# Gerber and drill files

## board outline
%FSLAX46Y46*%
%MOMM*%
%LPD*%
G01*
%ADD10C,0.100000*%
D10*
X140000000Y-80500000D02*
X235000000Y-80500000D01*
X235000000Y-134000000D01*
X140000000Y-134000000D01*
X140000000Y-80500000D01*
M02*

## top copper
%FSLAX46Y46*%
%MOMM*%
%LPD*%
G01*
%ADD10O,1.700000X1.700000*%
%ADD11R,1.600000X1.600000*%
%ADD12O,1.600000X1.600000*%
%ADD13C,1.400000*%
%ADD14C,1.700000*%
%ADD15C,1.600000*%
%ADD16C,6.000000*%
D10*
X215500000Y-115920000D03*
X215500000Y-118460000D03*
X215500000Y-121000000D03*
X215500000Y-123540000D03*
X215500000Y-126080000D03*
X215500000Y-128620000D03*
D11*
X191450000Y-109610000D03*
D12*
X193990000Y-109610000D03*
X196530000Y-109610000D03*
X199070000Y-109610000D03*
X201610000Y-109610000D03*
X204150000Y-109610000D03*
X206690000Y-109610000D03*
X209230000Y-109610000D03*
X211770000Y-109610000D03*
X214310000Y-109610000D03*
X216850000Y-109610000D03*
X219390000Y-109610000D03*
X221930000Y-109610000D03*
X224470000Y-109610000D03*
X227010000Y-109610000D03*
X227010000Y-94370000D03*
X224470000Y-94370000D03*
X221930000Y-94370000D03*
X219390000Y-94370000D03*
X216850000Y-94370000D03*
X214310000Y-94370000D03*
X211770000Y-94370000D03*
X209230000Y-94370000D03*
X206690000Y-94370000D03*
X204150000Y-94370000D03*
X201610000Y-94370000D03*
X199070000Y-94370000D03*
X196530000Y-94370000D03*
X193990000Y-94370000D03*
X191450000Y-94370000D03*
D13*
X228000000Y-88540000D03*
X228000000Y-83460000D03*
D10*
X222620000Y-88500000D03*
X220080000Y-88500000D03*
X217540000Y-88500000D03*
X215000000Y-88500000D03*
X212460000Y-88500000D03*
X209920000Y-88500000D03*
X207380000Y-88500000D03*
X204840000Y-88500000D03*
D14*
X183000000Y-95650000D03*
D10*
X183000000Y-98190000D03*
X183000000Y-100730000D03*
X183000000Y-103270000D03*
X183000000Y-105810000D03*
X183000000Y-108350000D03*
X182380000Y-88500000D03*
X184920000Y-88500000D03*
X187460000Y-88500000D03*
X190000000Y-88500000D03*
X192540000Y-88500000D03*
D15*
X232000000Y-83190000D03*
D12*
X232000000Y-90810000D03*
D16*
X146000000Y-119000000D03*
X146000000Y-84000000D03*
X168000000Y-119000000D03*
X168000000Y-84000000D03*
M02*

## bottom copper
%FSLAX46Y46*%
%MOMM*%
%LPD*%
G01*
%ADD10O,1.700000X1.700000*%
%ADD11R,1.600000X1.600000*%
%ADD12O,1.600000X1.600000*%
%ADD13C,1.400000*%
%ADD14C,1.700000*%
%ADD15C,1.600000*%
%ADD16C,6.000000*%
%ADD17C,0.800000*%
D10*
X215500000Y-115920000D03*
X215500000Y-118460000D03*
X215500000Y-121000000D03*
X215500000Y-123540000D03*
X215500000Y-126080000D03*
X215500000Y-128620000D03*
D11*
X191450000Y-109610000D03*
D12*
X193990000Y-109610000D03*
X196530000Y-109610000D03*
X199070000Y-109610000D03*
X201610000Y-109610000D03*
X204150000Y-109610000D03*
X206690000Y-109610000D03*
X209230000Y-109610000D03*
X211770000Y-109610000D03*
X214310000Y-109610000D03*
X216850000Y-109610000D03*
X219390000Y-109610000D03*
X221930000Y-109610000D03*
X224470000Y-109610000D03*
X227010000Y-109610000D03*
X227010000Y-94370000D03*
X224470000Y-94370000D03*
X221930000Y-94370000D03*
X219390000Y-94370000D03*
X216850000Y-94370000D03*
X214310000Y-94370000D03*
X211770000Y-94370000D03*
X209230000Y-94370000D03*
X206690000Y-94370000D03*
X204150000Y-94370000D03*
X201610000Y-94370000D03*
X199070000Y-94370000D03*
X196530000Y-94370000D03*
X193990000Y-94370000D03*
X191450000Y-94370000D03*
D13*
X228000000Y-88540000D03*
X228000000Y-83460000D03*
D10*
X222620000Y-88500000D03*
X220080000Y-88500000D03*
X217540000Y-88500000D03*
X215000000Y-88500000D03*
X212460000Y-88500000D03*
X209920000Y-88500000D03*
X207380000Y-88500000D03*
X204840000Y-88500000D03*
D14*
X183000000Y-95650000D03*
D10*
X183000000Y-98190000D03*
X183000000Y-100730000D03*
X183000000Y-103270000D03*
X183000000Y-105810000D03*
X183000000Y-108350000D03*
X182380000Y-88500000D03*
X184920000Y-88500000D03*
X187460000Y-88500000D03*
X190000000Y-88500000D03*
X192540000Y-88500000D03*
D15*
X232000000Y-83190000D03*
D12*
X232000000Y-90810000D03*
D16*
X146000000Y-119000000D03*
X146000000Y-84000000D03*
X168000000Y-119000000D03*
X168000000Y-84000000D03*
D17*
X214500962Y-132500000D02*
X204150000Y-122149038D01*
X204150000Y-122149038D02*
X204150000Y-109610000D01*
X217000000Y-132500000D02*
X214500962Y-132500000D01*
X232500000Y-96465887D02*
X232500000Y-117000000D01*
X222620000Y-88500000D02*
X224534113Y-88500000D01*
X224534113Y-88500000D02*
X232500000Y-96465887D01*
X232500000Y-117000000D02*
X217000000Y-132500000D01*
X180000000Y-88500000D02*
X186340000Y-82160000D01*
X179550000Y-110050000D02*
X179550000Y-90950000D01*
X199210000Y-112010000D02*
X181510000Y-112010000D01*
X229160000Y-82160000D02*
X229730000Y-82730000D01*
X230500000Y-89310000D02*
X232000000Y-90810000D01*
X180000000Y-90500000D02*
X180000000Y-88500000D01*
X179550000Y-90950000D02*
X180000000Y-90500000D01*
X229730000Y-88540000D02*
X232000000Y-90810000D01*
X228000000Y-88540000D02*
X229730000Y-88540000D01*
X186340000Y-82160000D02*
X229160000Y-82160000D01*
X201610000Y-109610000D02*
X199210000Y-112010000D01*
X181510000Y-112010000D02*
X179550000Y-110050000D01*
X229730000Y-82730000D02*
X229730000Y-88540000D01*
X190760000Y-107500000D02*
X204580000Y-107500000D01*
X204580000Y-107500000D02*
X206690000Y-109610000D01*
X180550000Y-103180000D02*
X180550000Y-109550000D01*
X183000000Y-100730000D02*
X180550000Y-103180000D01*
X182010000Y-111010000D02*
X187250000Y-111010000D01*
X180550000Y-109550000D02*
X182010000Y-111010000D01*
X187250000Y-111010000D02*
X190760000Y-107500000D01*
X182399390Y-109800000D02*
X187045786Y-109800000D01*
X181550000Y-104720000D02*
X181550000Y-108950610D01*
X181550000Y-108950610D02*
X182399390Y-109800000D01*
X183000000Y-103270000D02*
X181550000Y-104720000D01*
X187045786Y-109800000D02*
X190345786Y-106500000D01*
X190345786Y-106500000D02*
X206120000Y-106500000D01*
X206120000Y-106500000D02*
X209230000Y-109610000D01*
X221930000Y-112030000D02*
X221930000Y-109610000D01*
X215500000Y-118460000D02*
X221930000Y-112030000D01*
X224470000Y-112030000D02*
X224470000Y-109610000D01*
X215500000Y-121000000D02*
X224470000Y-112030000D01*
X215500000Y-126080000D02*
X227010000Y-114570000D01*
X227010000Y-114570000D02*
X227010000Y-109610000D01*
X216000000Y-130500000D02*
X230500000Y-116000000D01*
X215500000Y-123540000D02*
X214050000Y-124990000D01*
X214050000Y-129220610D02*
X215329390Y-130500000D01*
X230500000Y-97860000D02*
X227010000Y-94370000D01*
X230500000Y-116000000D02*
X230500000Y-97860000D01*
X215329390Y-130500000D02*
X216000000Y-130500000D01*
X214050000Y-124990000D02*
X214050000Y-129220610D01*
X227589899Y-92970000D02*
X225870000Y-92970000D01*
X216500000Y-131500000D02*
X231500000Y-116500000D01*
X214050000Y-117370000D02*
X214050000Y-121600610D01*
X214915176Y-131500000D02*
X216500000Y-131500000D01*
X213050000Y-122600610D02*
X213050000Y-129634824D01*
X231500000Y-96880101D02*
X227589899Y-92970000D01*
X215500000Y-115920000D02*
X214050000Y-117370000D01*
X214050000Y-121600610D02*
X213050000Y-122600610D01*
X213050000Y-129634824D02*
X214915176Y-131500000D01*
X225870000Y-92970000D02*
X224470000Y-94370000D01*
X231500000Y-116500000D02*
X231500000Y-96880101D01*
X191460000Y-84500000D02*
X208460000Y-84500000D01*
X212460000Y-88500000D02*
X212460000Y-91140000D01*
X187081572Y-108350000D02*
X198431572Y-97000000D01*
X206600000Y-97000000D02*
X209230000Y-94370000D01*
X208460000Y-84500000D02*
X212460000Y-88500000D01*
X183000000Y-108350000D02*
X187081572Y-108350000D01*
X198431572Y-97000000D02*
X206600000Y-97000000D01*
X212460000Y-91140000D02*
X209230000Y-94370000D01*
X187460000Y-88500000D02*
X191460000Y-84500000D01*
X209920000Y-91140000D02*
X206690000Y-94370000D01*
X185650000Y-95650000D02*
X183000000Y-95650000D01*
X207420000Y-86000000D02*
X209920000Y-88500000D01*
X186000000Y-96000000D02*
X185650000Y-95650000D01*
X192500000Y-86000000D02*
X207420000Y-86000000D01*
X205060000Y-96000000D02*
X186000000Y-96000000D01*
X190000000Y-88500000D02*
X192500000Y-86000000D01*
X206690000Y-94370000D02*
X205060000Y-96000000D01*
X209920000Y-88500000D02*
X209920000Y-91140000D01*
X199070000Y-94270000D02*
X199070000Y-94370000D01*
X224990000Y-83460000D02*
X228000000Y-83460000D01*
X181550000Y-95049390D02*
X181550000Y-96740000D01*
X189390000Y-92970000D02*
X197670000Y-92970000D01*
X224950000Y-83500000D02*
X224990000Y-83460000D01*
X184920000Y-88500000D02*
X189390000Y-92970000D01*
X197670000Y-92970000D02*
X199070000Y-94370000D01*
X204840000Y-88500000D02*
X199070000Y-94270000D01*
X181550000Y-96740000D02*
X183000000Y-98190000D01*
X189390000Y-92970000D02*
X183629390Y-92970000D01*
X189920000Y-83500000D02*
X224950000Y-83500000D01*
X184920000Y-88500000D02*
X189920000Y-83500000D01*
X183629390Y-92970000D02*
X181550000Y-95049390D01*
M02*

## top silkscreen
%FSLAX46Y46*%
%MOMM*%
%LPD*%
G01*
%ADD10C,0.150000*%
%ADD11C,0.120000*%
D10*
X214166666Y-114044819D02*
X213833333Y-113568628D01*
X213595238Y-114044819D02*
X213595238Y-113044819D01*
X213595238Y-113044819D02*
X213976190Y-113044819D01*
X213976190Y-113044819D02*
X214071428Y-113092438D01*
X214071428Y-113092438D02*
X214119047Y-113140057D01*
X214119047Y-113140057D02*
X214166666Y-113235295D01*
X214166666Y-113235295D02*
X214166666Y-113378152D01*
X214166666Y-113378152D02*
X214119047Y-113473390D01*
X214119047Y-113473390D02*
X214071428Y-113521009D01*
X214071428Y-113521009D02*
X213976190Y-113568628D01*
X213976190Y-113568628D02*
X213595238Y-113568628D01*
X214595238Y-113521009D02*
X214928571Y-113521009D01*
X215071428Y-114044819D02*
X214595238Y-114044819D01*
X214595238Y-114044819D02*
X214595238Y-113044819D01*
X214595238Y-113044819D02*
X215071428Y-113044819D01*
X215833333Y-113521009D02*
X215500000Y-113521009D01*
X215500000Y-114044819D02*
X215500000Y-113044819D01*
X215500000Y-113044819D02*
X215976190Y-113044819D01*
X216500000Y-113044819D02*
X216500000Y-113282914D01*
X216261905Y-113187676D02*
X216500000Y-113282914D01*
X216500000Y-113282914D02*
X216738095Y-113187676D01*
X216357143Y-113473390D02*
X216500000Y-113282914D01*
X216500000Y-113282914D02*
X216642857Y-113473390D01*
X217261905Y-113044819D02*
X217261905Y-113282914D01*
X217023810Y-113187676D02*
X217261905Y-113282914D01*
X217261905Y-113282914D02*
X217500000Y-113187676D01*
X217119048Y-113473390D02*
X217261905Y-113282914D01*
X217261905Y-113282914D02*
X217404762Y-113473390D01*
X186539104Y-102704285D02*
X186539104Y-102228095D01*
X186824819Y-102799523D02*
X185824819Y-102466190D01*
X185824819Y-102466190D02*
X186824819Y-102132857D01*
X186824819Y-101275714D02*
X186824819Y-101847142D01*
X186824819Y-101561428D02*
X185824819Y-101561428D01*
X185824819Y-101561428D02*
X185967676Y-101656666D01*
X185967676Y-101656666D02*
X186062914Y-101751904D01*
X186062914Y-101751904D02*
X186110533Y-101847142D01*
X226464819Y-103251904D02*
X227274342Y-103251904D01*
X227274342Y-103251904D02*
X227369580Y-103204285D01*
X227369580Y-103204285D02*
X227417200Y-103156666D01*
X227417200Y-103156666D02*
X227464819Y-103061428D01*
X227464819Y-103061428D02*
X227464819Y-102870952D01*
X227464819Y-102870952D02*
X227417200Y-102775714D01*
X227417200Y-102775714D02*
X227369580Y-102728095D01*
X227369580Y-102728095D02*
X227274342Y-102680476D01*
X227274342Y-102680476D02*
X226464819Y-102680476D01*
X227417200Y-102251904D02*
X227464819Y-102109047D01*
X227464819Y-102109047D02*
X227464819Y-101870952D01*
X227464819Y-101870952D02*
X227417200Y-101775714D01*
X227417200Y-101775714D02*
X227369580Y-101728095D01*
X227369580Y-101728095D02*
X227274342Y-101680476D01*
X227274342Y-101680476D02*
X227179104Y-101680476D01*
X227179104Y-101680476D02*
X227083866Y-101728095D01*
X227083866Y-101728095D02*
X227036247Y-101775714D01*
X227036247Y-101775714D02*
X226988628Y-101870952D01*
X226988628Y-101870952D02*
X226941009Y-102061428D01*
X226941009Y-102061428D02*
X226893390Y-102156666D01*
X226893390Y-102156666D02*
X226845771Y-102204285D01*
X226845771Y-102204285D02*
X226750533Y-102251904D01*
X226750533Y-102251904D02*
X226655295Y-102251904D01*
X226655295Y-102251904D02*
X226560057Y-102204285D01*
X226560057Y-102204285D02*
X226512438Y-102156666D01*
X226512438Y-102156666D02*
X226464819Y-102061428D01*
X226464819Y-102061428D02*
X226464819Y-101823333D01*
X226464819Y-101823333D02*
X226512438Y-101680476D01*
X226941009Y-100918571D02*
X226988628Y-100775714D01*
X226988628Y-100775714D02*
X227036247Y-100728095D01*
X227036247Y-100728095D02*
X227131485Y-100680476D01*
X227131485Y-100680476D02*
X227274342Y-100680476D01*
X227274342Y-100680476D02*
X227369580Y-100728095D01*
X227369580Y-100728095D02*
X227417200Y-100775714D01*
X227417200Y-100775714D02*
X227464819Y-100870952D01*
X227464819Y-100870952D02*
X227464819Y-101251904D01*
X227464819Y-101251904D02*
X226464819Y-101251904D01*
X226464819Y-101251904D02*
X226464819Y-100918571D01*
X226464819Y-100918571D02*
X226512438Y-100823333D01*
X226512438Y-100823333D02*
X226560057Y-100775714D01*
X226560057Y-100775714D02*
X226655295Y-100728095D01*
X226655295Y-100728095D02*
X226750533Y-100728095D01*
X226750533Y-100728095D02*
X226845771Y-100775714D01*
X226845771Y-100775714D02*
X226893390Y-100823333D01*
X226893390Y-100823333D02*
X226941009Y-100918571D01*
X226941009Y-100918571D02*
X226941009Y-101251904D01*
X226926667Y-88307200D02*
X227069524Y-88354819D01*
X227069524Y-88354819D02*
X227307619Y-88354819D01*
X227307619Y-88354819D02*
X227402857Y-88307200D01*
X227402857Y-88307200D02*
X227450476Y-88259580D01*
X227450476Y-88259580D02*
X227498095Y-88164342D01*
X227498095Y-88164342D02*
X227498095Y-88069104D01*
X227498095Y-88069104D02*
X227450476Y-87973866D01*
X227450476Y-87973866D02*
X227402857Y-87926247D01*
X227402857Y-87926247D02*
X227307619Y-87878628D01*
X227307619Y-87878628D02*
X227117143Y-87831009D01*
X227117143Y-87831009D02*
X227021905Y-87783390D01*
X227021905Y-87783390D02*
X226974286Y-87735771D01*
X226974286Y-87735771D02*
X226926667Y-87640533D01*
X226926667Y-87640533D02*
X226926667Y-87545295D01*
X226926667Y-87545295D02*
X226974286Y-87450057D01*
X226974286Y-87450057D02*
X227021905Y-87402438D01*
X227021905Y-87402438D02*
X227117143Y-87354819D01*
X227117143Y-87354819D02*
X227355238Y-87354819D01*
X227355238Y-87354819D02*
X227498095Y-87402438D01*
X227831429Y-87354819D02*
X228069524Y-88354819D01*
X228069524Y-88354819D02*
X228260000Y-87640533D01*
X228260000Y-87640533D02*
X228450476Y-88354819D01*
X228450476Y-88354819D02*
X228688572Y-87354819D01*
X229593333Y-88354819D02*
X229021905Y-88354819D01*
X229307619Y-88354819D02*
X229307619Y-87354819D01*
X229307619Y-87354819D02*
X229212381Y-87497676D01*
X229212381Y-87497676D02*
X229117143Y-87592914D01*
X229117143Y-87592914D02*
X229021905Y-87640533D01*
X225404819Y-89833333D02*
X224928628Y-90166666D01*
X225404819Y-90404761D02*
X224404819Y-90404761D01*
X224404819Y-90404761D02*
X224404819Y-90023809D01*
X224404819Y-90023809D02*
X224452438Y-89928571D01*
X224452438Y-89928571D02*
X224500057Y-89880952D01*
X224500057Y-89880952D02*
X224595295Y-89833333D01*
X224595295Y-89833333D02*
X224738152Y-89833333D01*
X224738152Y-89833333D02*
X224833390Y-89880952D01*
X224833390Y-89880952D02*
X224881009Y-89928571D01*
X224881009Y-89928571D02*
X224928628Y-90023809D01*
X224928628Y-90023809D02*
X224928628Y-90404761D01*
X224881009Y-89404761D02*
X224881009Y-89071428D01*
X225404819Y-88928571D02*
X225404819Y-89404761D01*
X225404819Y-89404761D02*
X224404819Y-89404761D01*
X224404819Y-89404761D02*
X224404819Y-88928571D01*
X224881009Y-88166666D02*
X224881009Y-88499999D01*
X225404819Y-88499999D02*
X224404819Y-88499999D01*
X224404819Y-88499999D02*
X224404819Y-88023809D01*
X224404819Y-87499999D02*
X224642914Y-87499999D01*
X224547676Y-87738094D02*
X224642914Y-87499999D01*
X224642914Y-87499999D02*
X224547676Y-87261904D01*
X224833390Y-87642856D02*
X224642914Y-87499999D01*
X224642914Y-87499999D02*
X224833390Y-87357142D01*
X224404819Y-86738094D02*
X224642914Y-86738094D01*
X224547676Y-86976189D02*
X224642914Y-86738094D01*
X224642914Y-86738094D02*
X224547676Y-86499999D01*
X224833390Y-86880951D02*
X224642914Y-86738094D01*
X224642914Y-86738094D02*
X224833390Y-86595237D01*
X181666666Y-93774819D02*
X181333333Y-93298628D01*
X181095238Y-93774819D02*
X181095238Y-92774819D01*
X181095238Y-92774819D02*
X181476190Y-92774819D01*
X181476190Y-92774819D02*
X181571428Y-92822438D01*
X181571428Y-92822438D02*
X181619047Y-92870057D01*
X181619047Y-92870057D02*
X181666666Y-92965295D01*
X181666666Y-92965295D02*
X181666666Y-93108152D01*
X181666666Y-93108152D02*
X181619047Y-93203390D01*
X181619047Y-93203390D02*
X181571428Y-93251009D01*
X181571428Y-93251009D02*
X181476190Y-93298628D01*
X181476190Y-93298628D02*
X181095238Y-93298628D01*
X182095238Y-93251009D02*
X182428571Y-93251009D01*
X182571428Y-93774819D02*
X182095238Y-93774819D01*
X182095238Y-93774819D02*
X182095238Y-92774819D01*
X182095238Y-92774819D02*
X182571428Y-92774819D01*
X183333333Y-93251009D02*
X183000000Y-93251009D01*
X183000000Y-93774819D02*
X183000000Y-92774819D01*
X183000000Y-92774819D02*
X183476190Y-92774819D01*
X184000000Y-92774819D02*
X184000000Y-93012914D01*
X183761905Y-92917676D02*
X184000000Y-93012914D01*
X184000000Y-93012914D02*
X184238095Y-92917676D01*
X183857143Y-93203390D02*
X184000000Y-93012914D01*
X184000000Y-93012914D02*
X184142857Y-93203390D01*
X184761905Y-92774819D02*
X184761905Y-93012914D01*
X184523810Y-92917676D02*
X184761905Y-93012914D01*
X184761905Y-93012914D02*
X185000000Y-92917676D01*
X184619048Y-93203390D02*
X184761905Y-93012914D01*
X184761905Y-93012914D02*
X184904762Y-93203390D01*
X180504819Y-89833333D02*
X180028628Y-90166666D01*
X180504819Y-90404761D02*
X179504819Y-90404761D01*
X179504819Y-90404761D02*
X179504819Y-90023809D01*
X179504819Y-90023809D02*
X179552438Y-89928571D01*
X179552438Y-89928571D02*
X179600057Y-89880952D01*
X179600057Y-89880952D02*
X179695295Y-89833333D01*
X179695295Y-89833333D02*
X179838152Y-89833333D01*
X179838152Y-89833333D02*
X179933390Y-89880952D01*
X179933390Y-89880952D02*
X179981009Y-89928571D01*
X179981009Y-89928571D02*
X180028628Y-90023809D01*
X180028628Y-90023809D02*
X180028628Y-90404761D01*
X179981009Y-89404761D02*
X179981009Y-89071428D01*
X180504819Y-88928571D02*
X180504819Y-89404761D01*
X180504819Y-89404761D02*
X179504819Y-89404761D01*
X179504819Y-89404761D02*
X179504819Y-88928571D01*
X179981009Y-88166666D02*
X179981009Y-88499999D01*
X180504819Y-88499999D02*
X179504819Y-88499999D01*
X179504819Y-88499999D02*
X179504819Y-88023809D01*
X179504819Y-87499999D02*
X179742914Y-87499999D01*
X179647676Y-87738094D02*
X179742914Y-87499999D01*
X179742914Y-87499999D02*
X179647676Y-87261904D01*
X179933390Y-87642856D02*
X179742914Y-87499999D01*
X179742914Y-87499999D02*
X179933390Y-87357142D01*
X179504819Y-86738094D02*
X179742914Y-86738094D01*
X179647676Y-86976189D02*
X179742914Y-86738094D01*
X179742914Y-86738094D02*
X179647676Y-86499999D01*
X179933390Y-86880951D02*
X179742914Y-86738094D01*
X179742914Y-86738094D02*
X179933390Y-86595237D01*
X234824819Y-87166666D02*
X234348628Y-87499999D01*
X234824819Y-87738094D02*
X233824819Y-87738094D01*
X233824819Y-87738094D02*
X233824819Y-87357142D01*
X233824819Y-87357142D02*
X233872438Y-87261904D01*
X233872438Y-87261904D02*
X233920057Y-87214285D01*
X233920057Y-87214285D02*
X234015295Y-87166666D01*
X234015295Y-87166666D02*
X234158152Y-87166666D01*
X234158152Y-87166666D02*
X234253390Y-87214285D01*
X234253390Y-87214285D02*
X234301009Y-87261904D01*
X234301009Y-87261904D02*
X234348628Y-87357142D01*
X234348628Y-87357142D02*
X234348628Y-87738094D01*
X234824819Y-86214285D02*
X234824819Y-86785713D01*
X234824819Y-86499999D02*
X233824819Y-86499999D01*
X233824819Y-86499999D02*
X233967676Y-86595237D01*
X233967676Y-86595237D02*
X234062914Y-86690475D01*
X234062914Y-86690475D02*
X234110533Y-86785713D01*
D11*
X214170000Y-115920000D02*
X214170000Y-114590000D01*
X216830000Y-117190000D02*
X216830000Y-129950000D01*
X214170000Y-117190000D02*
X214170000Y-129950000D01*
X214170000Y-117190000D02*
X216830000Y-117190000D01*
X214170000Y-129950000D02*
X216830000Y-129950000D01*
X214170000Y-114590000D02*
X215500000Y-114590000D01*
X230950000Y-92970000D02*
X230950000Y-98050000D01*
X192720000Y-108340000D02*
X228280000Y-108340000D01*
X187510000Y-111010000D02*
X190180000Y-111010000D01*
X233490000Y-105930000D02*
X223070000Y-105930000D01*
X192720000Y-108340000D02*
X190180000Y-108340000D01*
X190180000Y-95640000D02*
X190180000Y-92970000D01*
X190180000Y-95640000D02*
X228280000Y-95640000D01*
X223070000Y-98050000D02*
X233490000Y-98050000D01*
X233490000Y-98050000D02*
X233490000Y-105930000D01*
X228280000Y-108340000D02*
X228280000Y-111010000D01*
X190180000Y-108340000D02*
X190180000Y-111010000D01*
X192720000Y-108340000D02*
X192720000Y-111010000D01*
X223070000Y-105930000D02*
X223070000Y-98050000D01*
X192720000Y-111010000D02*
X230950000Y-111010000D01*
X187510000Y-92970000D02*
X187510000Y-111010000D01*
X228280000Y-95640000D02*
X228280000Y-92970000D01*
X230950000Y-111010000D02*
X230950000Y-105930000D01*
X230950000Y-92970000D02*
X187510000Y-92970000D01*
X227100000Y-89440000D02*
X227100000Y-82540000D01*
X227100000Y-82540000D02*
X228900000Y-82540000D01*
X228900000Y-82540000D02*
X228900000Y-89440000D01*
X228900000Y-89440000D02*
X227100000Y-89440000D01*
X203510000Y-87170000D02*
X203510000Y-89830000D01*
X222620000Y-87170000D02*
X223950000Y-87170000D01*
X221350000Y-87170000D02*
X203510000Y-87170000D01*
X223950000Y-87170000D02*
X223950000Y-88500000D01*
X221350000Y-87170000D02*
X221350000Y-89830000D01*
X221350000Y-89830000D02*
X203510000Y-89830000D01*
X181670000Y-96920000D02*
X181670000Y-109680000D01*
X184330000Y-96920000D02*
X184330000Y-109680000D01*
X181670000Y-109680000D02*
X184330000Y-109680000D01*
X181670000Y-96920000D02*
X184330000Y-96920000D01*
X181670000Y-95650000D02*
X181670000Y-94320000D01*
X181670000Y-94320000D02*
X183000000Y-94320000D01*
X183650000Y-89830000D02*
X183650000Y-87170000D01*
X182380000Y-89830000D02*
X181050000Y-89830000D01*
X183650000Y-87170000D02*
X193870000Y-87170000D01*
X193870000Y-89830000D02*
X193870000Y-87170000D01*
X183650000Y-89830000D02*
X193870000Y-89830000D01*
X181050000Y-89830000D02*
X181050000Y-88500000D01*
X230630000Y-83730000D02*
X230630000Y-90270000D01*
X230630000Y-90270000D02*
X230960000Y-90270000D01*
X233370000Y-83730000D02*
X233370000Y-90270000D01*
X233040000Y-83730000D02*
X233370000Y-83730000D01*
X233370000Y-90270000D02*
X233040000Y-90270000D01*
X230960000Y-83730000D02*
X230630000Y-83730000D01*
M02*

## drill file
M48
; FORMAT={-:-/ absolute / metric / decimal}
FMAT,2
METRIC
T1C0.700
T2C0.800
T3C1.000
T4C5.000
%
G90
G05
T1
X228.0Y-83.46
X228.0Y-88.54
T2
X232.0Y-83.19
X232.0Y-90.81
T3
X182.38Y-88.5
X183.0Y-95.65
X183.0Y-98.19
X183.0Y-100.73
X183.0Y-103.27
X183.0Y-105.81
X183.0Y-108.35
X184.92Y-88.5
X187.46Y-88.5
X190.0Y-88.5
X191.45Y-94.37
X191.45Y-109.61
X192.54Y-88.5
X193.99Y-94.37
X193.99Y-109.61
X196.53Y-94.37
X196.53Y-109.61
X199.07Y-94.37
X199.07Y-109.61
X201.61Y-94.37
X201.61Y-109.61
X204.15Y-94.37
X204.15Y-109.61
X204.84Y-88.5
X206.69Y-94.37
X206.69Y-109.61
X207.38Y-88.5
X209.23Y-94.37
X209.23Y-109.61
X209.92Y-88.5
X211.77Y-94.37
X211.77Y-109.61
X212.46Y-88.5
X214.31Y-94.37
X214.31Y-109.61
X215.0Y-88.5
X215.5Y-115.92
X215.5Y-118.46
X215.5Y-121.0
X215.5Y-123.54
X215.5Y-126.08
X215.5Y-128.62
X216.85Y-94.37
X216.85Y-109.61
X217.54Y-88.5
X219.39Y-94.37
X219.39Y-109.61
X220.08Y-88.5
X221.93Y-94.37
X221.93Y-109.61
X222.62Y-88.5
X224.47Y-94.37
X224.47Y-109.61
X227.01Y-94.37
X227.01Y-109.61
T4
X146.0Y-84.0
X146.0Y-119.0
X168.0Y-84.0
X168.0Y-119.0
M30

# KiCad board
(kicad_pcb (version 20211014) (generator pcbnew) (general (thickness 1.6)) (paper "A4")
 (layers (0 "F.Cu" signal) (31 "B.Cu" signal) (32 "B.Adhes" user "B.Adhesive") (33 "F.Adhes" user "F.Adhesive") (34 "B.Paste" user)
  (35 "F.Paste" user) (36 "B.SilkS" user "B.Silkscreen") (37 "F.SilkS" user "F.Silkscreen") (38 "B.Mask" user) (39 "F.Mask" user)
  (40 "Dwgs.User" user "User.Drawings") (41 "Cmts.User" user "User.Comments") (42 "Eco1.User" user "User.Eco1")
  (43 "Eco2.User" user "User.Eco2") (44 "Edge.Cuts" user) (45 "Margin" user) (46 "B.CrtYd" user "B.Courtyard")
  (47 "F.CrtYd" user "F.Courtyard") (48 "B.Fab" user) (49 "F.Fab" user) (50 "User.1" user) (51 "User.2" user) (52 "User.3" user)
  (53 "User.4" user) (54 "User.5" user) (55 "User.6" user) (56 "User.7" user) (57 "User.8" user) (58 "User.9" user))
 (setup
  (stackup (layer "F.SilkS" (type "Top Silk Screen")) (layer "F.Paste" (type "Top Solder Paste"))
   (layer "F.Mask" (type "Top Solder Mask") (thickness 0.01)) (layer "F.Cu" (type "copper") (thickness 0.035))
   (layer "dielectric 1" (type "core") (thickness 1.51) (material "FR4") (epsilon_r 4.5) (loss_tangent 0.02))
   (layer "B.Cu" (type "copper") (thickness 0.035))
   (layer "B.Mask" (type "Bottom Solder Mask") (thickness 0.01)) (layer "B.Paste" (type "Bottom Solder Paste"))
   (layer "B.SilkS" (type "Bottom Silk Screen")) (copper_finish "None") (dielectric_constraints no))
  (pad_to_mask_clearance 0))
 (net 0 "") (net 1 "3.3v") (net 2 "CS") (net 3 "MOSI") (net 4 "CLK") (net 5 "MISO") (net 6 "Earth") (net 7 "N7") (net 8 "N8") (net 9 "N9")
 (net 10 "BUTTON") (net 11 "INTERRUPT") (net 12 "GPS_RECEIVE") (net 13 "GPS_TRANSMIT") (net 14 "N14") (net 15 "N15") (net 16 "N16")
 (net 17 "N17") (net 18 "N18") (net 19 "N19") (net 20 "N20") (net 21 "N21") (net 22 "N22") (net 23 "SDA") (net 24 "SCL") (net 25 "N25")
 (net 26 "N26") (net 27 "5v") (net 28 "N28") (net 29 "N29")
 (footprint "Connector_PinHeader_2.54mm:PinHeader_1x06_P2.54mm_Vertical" (layer "F.Cu") (at 215.5 115.92)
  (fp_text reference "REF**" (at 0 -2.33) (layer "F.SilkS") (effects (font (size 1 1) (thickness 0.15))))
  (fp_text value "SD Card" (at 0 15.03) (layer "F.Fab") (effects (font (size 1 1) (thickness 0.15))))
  (fp_line (start -1.33 0) (end -1.33 -1.33) (layer "F.SilkS") (width 0.12))
  (fp_line (start 1.33 1.27) (end 1.33 14.03) (layer "F.SilkS") (width 0.12))
  (fp_line (start -1.33 1.27) (end -1.33 14.03) (layer "F.SilkS") (width 0.12))
  (fp_line (start -1.33 1.27) (end 1.33 1.27) (layer "F.SilkS") (width 0.12))
  (fp_line (start -1.33 14.03) (end 1.33 14.03) (layer "F.SilkS") (width 0.12))
  (fp_line (start -1.33 -1.33) (end 0 -1.33) (layer "F.SilkS") (width 0.12))
  (pad "1" thru_hole oval (at 0 0) (size 1.7 1.7) (drill 1) (layers *.Cu *.Mask) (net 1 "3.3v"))
  (pad "2" thru_hole oval (at 0 2.54) (size 1.7 1.7) (drill 1) (layers *.Cu *.Mask) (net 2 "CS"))
  (pad "3" thru_hole oval (at 0 5.08) (size 1.7 1.7) (drill 1) (layers *.Cu *.Mask) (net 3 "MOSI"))
  (pad "4" thru_hole oval (at 0 7.62) (size 1.7 1.7) (drill 1) (layers *.Cu *.Mask) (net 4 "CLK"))
  (pad "5" thru_hole oval (at 0 10.16) (size 1.7 1.7) (drill 1) (layers *.Cu *.Mask) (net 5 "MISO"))
  (pad "6" thru_hole oval (at 0 12.7) (size 1.7 1.7) (drill 1) (layers *.Cu *.Mask) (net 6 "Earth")))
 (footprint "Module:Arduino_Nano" (layer "F.Cu") (at 191.45 109.61 90)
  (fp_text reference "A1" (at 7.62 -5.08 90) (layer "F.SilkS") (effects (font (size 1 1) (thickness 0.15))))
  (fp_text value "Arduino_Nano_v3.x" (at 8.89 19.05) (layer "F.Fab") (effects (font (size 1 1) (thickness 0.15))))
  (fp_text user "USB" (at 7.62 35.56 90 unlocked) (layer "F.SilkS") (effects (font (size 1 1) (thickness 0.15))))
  (fp_line (start 16.64 39.5) (end 11.56 39.5) (layer "F.SilkS") (width 0.12))
  (fp_line (start 1.27 1.27) (end 1.27 36.83) (layer "F.SilkS") (width 0.12))
  (fp_line (start -1.4 -3.94) (end -1.4 -1.27) (layer "F.SilkS") (width 0.12))
  (fp_line (start 3.68 42.04) (end 3.68 31.62) (layer "F.SilkS") (width 0.12))
  (fp_line (start 1.27 1.27) (end 1.27 -1.27) (layer "F.SilkS") (width 0.12))
  (fp_line (start 13.97 -1.27) (end 16.64 -1.27) (layer "F.SilkS") (width 0.12))
  (fp_line (start 13.97 -1.27) (end 13.97 36.83) (layer "F.SilkS") (width 0.12))
  (fp_line (start 11.56 31.62) (end 11.56 42.04) (layer "F.SilkS") (width 0.12))
  (fp_line (start 11.56 42.04) (end 3.68 42.04) (layer "F.SilkS") (width 0.12))
  (fp_line (start 1.27 36.83) (end -1.4 36.83) (layer "F.SilkS") (width 0.12))
  (fp_line (start 1.27 -1.27) (end -1.4 -1.27) (layer "F.SilkS") (width 0.12))
  (fp_line (start 1.27 1.27) (end -1.4 1.27) (layer "F.SilkS") (width 0.12))
  (fp_line (start 3.68 31.62) (end 11.56 31.62) (layer "F.SilkS") (width 0.12))
  (fp_line (start -1.4 1.27) (end -1.4 39.5) (layer "F.SilkS") (width 0.12))
  (fp_line (start 16.64 -3.94) (end -1.4 -3.94) (layer "F.SilkS") (width 0.12))
  (fp_line (start 13.97 36.83) (end 16.64 36.83) (layer "F.SilkS") (width 0.12))
  (fp_line (start -1.4 39.5) (end 3.68 39.5) (layer "F.SilkS") (width 0.12))
  (fp_line (start 16.64 39.5) (end 16.64 -3.94) (layer "F.SilkS") (width 0.12))
  (pad "1" thru_hole rect (at 0 0 90) (size 1.6 1.6) (drill 1) (layers *.Cu *.Mask) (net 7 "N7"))
  (pad "2" thru_hole oval (at 0 2.54 90) (size 1.6 1.6) (drill 1) (layers *.Cu *.Mask) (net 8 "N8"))
  (pad "3" thru_hole oval (at 0 5.08 90) (size 1.6 1.6) (drill 1) (layers *.Cu *.Mask) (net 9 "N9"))
  (pad "4" thru_hole oval (at 0 7.62 90) (size 1.6 1.6) (drill 1) (layers *.Cu *.Mask) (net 6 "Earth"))
  (pad "5" thru_hole oval (at 0 10.16 90) (size 1.6 1.6) (drill 1) (layers *.Cu *.Mask) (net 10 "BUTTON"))
  (pad "6" thru_hole oval (at 0 12.7 90) (size 1.6 1.6) (drill 1) (layers *.Cu *.Mask) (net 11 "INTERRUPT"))
  (pad "7" thru_hole oval (at 0 15.24 90) (size 1.6 1.6) (drill 1) (layers *.Cu *.Mask) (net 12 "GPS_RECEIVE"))
  (pad "8" thru_hole oval (at 0 17.78 90) (size 1.6 1.6) (drill 1) (layers *.Cu *.Mask) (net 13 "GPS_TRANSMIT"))
  (pad "9" thru_hole oval (at 0 20.32 90) (size 1.6 1.6) (drill 1) (layers *.Cu *.Mask) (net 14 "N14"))
  (pad "10" thru_hole oval (at 0 22.86 90) (size 1.6 1.6) (drill 1) (layers *.Cu *.Mask) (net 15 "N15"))
  (pad "11" thru_hole oval (at 0 25.4 90) (size 1.6 1.6) (drill 1) (layers *.Cu *.Mask) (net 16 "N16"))
  (pad "12" thru_hole oval (at 0 27.94 90) (size 1.6 1.6) (drill 1) (layers *.Cu *.Mask) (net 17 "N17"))
  (pad "13" thru_hole oval (at 0 30.48 90) (size 1.6 1.6) (drill 1) (layers *.Cu *.Mask) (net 2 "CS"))
  (pad "14" thru_hole oval (at 0 33.02 90) (size 1.6 1.6) (drill 1) (layers *.Cu *.Mask) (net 3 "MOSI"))
  (pad "15" thru_hole oval (at 0 35.56 90) (size 1.6 1.6) (drill 1) (layers *.Cu *.Mask) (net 5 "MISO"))
  (pad "16" thru_hole oval (at 15.24 35.56 90) (size 1.6 1.6) (drill 1) (layers *.Cu *.Mask) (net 4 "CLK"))
  (pad "17" thru_hole oval (at 15.24 33.02 90) (size 1.6 1.6) (drill 1) (layers *.Cu *.Mask) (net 1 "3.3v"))
  (pad "18" thru_hole oval (at 15.24 30.48 90) (size 1.6 1.6) (drill 1) (layers *.Cu *.Mask) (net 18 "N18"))
  (pad "19" thru_hole oval (at 15.24 27.94 90) (size 1.6 1.6) (drill 1) (layers *.Cu *.Mask) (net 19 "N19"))
  (pad "20" thru_hole oval (at 15.24 25.4 90) (size 1.6 1.6) (drill 1) (layers *.Cu *.Mask) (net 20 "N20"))
  (pad "21" thru_hole oval (at 15.24 22.86 90) (size 1.6 1.6) (drill 1) (layers *.Cu *.Mask) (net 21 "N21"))
  (pad "22" thru_hole oval (at 15.24 20.32 90) (size 1.6 1.6) (drill 1) (layers *.Cu *.Mask) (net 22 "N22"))
  (pad "23" thru_hole oval (at 15.24 17.78 90) (size 1.6 1.6) (drill 1) (layers *.Cu *.Mask) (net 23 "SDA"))
  (pad "24" thru_hole oval (at 15.24 15.24 90) (size 1.6 1.6) (drill 1) (layers *.Cu *.Mask) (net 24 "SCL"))
  (pad "25" thru_hole oval (at 15.24 12.7 90) (size 1.6 1.6) (drill 1) (layers *.Cu *.Mask) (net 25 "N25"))
  (pad "26" thru_hole oval (at 15.24 10.16 90) (size 1.6 1.6) (drill 1) (layers *.Cu *.Mask) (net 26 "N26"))
  (pad "27" thru_hole oval (at 15.24 7.62 90) (size 1.6 1.6) (drill 1) (layers *.Cu *.Mask) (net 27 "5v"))
  (pad "28" thru_hole oval (at 15.24 5.08 90) (size 1.6 1.6) (drill 1) (layers *.Cu *.Mask) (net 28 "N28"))
  (pad "29" thru_hole oval (at 15.24 2.54 90) (size 1.6 1.6) (drill 1) (layers *.Cu *.Mask) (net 6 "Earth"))
  (pad "30" thru_hole oval (at 15.24 0 90) (size 1.6 1.6) (drill 1) (layers *.Cu *.Mask) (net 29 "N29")))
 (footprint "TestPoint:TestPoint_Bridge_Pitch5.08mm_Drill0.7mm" (layer "F.Cu") (at 228 88.54 90)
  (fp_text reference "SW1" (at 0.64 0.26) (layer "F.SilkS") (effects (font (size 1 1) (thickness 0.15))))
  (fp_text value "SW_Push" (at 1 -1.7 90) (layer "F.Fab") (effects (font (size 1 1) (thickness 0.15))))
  (fp_line (start -0.9 -0.9) (end 6 -0.9) (layer "F.SilkS") (width 0.12))
  (fp_line (start 6 -0.9) (end 6 0.9) (layer "F.SilkS") (width 0.12))
  (fp_line (start 6 0.9) (end -0.9 0.9) (layer "F.SilkS") (width 0.12))
  (fp_line (start -0.9 0.9) (end -0.9 -0.9) (layer "F.SilkS") (width 0.12))
  (pad "1" thru_hole circle (at 0 0 90) (size 1.4 1.4) (drill 0.7) (layers *.Cu *.Mask) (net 10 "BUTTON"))
  (pad "1" thru_hole circle (at 5.08 0 90) (size 1.4 1.4) (drill 0.7) (layers *.Cu *.Mask) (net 27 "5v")))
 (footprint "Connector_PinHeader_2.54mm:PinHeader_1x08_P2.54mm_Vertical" (layer "F.Cu") (at 222.62 88.5 -90)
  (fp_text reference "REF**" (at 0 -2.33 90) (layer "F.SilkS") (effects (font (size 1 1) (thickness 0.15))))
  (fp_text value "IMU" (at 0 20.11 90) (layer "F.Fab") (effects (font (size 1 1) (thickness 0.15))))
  (fp_line (start -1.33 19.11) (end 1.33 19.11) (layer "F.SilkS") (width 0.12))
  (fp_line (start -1.33 0) (end -1.33 -1.33) (layer "F.SilkS") (width 0.12))
  (fp_line (start -1.33 1.27) (end -1.33 19.11) (layer "F.SilkS") (width 0.12))
  (fp_line (start -1.33 -1.33) (end 0 -1.33) (layer "F.SilkS") (width 0.12))
  (fp_line (start -1.33 1.27) (end 1.33 1.27) (layer "F.SilkS") (width 0.12))
  (fp_line (start 1.33 1.27) (end 1.33 19.11) (layer "F.SilkS") (width 0.12))
  (pad "1" thru_hole oval (at 0 0 270) (size 1.7 1.7) (drill 1) (layers *.Cu *.Mask) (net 11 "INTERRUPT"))
  (pad "2" thru_hole oval (at 0 2.54 270) (size 1.7 1.7) (drill 1) (layers *.Cu *.Mask))
  (pad "3" thru_hole oval (at 0 5.08 270) (size 1.7 1.7) (drill 1) (layers *.Cu *.Mask))
  (pad "4" thru_hole oval (at 0 7.62 270) (size 1.7 1.7) (drill 1) (layers *.Cu *.Mask))
  (pad "5" thru_hole oval (at 0 10.16 270) (size 1.7 1.7) (drill 1) (layers *.Cu *.Mask) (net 23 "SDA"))
  (pad "6" thru_hole oval (at 0 12.7 270) (size 1.7 1.7) (drill 1) (layers *.Cu *.Mask) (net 24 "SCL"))
  (pad "7" thru_hole oval (at 0 15.24 270) (size 1.7 1.7) (drill 1) (layers *.Cu *.Mask) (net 6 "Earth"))
  (pad "8" thru_hole oval (at 0 17.78 270) (size 1.7 1.7) (drill 1) (layers *.Cu *.Mask) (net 27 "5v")))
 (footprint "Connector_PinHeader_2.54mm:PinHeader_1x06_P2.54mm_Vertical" (layer "F.Cu") (at 183 95.65)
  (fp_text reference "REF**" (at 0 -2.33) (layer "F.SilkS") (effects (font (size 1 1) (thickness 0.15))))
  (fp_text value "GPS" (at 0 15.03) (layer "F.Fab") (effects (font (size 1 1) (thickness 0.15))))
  (fp_line (start -1.33 1.27) (end -1.33 14.03) (layer "F.SilkS") (width 0.12))
  (fp_line (start 1.33 1.27) (end 1.33 14.03) (layer "F.SilkS") (width 0.12))
  (fp_line (start -1.33 14.03) (end 1.33 14.03) (layer "F.SilkS") (width 0.12))
  (fp_line (start -1.33 1.27) (end 1.33 1.27) (layer "F.SilkS") (width 0.12))
  (fp_line (start -1.33 0) (end -1.33 -1.33) (layer "F.SilkS") (width 0.12))
  (fp_line (start -1.33 -1.33) (end 0 -1.33) (layer "F.SilkS") (width 0.12))
  (pad "1" thru_hole circle (at 0 0) (size 1.7 1.7) (drill 1) (layers *.Cu *.Mask) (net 24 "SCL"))
  (pad "2" thru_hole oval (at 0 2.54) (size 1.7 1.7) (drill 1) (layers *.Cu *.Mask) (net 27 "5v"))
  (pad "3" thru_hole oval (at 0 5.08) (size 1.7 1.7) (drill 1) (layers *.Cu *.Mask) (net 12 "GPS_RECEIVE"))
  (pad "4" thru_hole oval (at 0 7.62) (size 1.7 1.7) (drill 1) (layers *.Cu *.Mask) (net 13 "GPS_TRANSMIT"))
  (pad "5" thru_hole oval (at 0 10.16) (size 1.7 1.7) (drill 1) (layers *.Cu *.Mask) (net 6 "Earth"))
  (pad "6" thru_hole oval (at 0 12.7) (size 1.7 1.7) (drill 1) (layers *.Cu *.Mask) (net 23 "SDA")))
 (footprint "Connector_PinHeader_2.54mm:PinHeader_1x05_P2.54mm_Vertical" (layer "F.Cu") (at 182.38 88.5 90)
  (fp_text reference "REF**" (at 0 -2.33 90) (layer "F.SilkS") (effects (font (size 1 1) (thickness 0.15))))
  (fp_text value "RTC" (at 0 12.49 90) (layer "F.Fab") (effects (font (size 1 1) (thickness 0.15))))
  (fp_line (start -1.33 1.27) (end 1.33 1.27) (layer "F.SilkS") (width 0.12))
  (fp_line (start -1.33 0) (end -1.33 -1.33) (layer "F.SilkS") (width 0.12))
  (fp_line (start 1.33 1.27) (end 1.33 11.49) (layer "F.SilkS") (width 0.12))
  (fp_line (start -1.33 11.49) (end 1.33 11.49) (layer "F.SilkS") (width 0.12))
  (fp_line (start -1.33 1.27) (end -1.33 11.49) (layer "F.SilkS") (width 0.12))
  (fp_line (start -1.33 -1.33) (end 0 -1.33) (layer "F.SilkS") (width 0.12))
  (pad "1" thru_hole oval (at 0 0 90) (size 1.7 1.7) (drill 1) (layers *.Cu *.Mask) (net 6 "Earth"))
  (pad "2" thru_hole oval (at 0 2.54 90) (size 1.7 1.7) (drill 1) (layers *.Cu *.Mask) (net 27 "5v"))
  (pad "3" thru_hole oval (at 0 5.08 90) (size 1.7 1.7) (drill 1) (layers *.Cu *.Mask) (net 23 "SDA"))
  (pad "4" thru_hole oval (at 0 7.62 90) (size 1.7 1.7) (drill 1) (layers *.Cu *.Mask) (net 24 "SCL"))
  (pad "5" thru_hole oval (at 0 10.16 90) (size 1.7 1.7) (drill 1) (layers *.Cu *.Mask)))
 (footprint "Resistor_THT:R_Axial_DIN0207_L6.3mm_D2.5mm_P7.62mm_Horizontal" (layer "F.Cu") (at 232 83.19 -90)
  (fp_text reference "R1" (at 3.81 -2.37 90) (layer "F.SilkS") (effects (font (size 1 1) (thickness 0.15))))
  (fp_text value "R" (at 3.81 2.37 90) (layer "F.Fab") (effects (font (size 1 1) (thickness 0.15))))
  (fp_line (start 0.54 1.37) (end 7.08 1.37) (layer "F.SilkS") (width 0.12))
  (fp_line (start 7.08 1.37) (end 7.08 1.04) (layer "F.SilkS") (width 0.12))
  (fp_line (start 0.54 -1.37) (end 7.08 -1.37) (layer "F.SilkS") (width 0.12))
  (fp_line (start 0.54 -1.04) (end 0.54 -1.37) (layer "F.SilkS") (width 0.12))
  (fp_line (start 7.08 -1.37) (end 7.08 -1.04) (layer "F.SilkS") (width 0.12))
  (fp_line (start 0.54 1.04) (end 0.54 1.37) (layer "F.SilkS") (width 0.12))
  (pad "1" thru_hole circle (at 0 0 270) (size 1.6 1.6) (drill 0.8) (layers *.Cu *.Mask) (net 6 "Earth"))
  (pad "2" thru_hole oval (at 7.62 0 270) (size 1.6 1.6) (drill 0.8) (layers *.Cu *.Mask) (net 10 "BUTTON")))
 (gr_rect (start 140 80.5) (end 235 134) (layer "Edge.Cuts") (width 0.1) (fill none))
 (via (at 146 119) (size 6) (drill 5) (layers "F.Cu" "B.Cu") (free) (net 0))
 (via (at 146 84) (size 6) (drill 5) (layers "F.Cu" "B.Cu") (free) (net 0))
 (via (at 168 119) (size 6) (drill 5) (layers "F.Cu" "B.Cu") (free) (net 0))
 (via (at 168 84) (size 6) (drill 5) (layers "F.Cu" "B.Cu") (free) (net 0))
 (segment (start 214.500962 132.5) (end 204.15 122.149038) (width 0.8) (layer "B.Cu") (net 11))
 (segment (start 204.15 122.149038) (end 204.15 109.61) (width 0.8) (layer "B.Cu") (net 11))
 (segment (start 217 132.5) (end 214.500962 132.5) (width 0.8) (layer "B.Cu") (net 11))
 (segment (start 232.5 96.465887) (end 232.5 117) (width 0.8) (layer "B.Cu") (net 11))
 (segment (start 222.62 88.5) (end 224.534113 88.5) (width 0.8) (layer "B.Cu") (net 11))
 (segment (start 224.534113 88.5) (end 232.5 96.465887) (width 0.8) (layer "B.Cu") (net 11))
 (segment (start 232.5 117) (end 217 132.5) (width 0.8) (layer "B.Cu") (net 11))
 (segment (start 180 88.5) (end 186.34 82.16) (width 0.8) (layer "B.Cu") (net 10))
 (segment (start 179.55 110.05) (end 179.55 90.95) (width 0.8) (layer "B.Cu") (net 10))
 (segment (start 199.21 112.01) (end 181.51 112.01) (width 0.8) (layer "B.Cu") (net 10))
 (segment (start 229.16 82.16) (end 229.73 82.73) (width 0.8) (layer "B.Cu") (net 10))
 (segment (start 230.5 89.31) (end 232 90.81) (width 0.8) (layer "B.Cu") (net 10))
 (segment (start 180 90.5) (end 180 88.5) (width 0.8) (layer "B.Cu") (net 10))
 (segment (start 179.55 90.95) (end 180 90.5) (width 0.8) (layer "B.Cu") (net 10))
 (segment (start 229.73 88.54) (end 232 90.81) (width 0.8) (layer "B.Cu") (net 10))
 (segment (start 228 88.54) (end 229.73 88.54) (width 0.8) (layer "B.Cu") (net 10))
 (segment (start 186.34 82.16) (end 229.16 82.16) (width 0.8) (layer "B.Cu") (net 10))
 (segment (start 201.61 109.61) (end 199.21 112.01) (width 0.8) (layer "B.Cu") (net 10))
 (segment (start 181.51 112.01) (end 179.55 110.05) (width 0.8) (layer "B.Cu") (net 10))
 (segment (start 229.73 82.73) (end 229.73 88.54) (width 0.8) (layer "B.Cu") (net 10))
 (segment (start 190.76 107.5) (end 204.58 107.5) (width 0.8) (layer "B.Cu") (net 12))
 (segment (start 204.58 107.5) (end 206.69 109.61) (width 0.8) (layer "B.Cu") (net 12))
 (segment (start 180.55 103.18) (end 180.55 109.55) (width 0.8) (layer "B.Cu") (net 12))
 (segment (start 183 100.73) (end 180.55 103.18) (width 0.8) (layer "B.Cu") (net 12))
 (segment (start 182.01 111.01) (end 187.25 111.01) (width 0.8) (layer "B.Cu") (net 12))
 (segment (start 180.55 109.55) (end 182.01 111.01) (width 0.8) (layer "B.Cu") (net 12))
 (segment (start 187.25 111.01) (end 190.76 107.5) (width 0.8) (layer "B.Cu") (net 12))
 (segment (start 182.39939 109.8) (end 187.045786 109.8) (width 0.8) (layer "B.Cu") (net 13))
 (segment (start 181.55 104.72) (end 181.55 108.95061) (width 0.8) (layer "B.Cu") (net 13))
 (segment (start 181.55 108.95061) (end 182.39939 109.8) (width 0.8) (layer "B.Cu") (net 13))
 (segment (start 183 103.27) (end 181.55 104.72) (width 0.8) (layer "B.Cu") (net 13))
 (segment (start 187.045786 109.8) (end 190.345786 106.5) (width 0.8) (layer "B.Cu") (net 13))
 (segment (start 190.345786 106.5) (end 206.12 106.5) (width 0.8) (layer "B.Cu") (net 13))
 (segment (start 206.12 106.5) (end 209.23 109.61) (width 0.8) (layer "B.Cu") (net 13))
 (segment (start 221.93 112.03) (end 221.93 109.61) (width 0.8) (layer "B.Cu") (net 2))
 (segment (start 215.5 118.46) (end 221.93 112.03) (width 0.8) (layer "B.Cu") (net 2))
 (segment (start 224.47 112.03) (end 224.47 109.61) (width 0.8) (layer "B.Cu") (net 3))
 (segment (start 215.5 121) (end 224.47 112.03) (width 0.8) (layer "B.Cu") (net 3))
 (segment (start 215.5 126.08) (end 227.01 114.57) (width 0.8) (layer "B.Cu") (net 5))
 (segment (start 227.01 114.57) (end 227.01 109.61) (width 0.8) (layer "B.Cu") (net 5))
 (segment (start 216 130.5) (end 230.5 116) (width 0.8) (layer "B.Cu") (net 4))
 (segment (start 215.5 123.54) (end 214.05 124.99) (width 0.8) (layer "B.Cu") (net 4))
 (segment (start 214.05 129.22061) (end 215.32939 130.5) (width 0.8) (layer "B.Cu") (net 4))
 (segment (start 230.5 97.86) (end 227.01 94.37) (width 0.8) (layer "B.Cu") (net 4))
 (segment (start 230.5 116) (end 230.5 97.86) (width 0.8) (layer "B.Cu") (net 4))
 (segment (start 215.32939 130.5) (end 216 130.5) (width 0.8) (layer "B.Cu") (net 4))
 (segment (start 214.05 124.99) (end 214.05 129.22061) (width 0.8) (layer "B.Cu") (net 4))
 (segment (start 227.589899 92.97) (end 225.87 92.97) (width 0.8) (layer "B.Cu") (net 1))
 (segment (start 216.5 131.5) (end 231.5 116.5) (width 0.8) (layer "B.Cu") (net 1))
 (segment (start 214.05 117.37) (end 214.05 121.60061) (width 0.8) (layer "B.Cu") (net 1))
 (segment (start 214.915176 131.5) (end 216.5 131.5) (width 0.8) (layer "B.Cu") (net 1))
 (segment (start 213.05 122.60061) (end 213.05 129.634824) (width 0.8) (layer "B.Cu") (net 1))
 (segment (start 231.5 96.880101) (end 227.589899 92.97) (width 0.8) (layer "B.Cu") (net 1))
 (segment (start 215.5 115.92) (end 214.05 117.37) (width 0.8) (layer "B.Cu") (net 1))
 (segment (start 214.05 121.60061) (end 213.05 122.60061) (width 0.8) (layer "B.Cu") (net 1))
 (segment (start 213.05 129.634824) (end 214.915176 131.5) (width 0.8) (layer "B.Cu") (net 1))
 (segment (start 225.87 92.97) (end 224.47 94.37) (width 0.8) (layer "B.Cu") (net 1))
 (segment (start 231.5 116.5) (end 231.5 96.880101) (width 0.8) (layer "B.Cu") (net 1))
 (segment (start 191.46 84.5) (end 208.46 84.5) (width 0.8) (layer "B.Cu") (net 23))
 (segment (start 212.46 88.5) (end 212.46 91.14) (width 0.8) (layer "B.Cu") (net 23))
 (segment (start 187.081572 108.35) (end 198.431572 97) (width 0.8) (layer "B.Cu") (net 23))
 (segment (start 206.6 97) (end 209.23 94.37) (width 0.8) (layer "B.Cu") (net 23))
 (segment (start 208.46 84.5) (end 212.46 88.5) (width 0.8) (layer "B.Cu") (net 23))
 (segment (start 183 108.35) (end 187.081572 108.35) (width 0.8) (layer "B.Cu") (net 23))
 (segment (start 198.431572 97) (end 206.6 97) (width 0.8) (layer "B.Cu") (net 23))
 (segment (start 212.46 91.14) (end 209.23 94.37) (width 0.8) (layer "B.Cu") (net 23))
 (segment (start 187.46 88.5) (end 191.46 84.5) (width 0.8) (layer "B.Cu") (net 23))
 (segment (start 209.92 91.14) (end 206.69 94.37) (width 0.8) (layer "B.Cu") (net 24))
 (segment (start 185.65 95.65) (end 183 95.65) (width 0.8) (layer "B.Cu") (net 24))
 (segment (start 207.42 86) (end 209.92 88.5) (width 0.8) (layer "B.Cu") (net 24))
 (segment (start 186 96) (end 185.65 95.65) (width 0.8) (layer "B.Cu") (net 24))
 (segment (start 192.5 86) (end 207.42 86) (width 0.8) (layer "B.Cu") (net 24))
 (segment (start 205.06 96) (end 186 96) (width 0.8) (layer "B.Cu") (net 24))
 (segment (start 190 88.5) (end 192.5 86) (width 0.8) (layer "B.Cu") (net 24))
 (segment (start 206.69 94.37) (end 205.06 96) (width 0.8) (layer "B.Cu") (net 24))
 (segment (start 209.92 88.5) (end 209.92 91.14) (width 0.8) (layer "B.Cu") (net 24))
 (segment (start 199.07 94.27) (end 199.07 94.37) (width 0.8) (layer "B.Cu") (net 27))
 (segment (start 224.99 83.46) (end 228 83.46) (width 0.8) (layer "B.Cu") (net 27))
 (segment (start 181.55 95.04939) (end 181.55 96.74) (width 0.8) (layer "B.Cu") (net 27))
 (segment (start 189.39 92.97) (end 197.67 92.97) (width 0.8) (layer "B.Cu") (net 27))
 (segment (start 224.95 83.5) (end 224.99 83.46) (width 0.8) (layer "B.Cu") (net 27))
 (segment (start 184.92 88.5) (end 189.39 92.97) (width 0.8) (layer "B.Cu") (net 27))
 (segment (start 197.67 92.97) (end 199.07 94.37) (width 0.8) (layer "B.Cu") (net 27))
 (segment (start 204.84 88.5) (end 199.07 94.27) (width 0.8) (layer "B.Cu") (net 27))
 (segment (start 181.55 96.74) (end 183 98.19) (width 0.8) (layer "B.Cu") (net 27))
 (segment (start 189.39 92.97) (end 183.62939 92.97) (width 0.8) (layer "B.Cu") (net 27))
 (segment (start 189.92 83.5) (end 224.95 83.5) (width 0.8) (layer "B.Cu") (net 27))
 (segment (start 184.92 88.5) (end 189.92 83.5) (width 0.8) (layer "B.Cu") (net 27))
 (segment (start 183.62939 92.97) (end 181.55 95.04939) (width 0.8) (layer "B.Cu") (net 27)))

